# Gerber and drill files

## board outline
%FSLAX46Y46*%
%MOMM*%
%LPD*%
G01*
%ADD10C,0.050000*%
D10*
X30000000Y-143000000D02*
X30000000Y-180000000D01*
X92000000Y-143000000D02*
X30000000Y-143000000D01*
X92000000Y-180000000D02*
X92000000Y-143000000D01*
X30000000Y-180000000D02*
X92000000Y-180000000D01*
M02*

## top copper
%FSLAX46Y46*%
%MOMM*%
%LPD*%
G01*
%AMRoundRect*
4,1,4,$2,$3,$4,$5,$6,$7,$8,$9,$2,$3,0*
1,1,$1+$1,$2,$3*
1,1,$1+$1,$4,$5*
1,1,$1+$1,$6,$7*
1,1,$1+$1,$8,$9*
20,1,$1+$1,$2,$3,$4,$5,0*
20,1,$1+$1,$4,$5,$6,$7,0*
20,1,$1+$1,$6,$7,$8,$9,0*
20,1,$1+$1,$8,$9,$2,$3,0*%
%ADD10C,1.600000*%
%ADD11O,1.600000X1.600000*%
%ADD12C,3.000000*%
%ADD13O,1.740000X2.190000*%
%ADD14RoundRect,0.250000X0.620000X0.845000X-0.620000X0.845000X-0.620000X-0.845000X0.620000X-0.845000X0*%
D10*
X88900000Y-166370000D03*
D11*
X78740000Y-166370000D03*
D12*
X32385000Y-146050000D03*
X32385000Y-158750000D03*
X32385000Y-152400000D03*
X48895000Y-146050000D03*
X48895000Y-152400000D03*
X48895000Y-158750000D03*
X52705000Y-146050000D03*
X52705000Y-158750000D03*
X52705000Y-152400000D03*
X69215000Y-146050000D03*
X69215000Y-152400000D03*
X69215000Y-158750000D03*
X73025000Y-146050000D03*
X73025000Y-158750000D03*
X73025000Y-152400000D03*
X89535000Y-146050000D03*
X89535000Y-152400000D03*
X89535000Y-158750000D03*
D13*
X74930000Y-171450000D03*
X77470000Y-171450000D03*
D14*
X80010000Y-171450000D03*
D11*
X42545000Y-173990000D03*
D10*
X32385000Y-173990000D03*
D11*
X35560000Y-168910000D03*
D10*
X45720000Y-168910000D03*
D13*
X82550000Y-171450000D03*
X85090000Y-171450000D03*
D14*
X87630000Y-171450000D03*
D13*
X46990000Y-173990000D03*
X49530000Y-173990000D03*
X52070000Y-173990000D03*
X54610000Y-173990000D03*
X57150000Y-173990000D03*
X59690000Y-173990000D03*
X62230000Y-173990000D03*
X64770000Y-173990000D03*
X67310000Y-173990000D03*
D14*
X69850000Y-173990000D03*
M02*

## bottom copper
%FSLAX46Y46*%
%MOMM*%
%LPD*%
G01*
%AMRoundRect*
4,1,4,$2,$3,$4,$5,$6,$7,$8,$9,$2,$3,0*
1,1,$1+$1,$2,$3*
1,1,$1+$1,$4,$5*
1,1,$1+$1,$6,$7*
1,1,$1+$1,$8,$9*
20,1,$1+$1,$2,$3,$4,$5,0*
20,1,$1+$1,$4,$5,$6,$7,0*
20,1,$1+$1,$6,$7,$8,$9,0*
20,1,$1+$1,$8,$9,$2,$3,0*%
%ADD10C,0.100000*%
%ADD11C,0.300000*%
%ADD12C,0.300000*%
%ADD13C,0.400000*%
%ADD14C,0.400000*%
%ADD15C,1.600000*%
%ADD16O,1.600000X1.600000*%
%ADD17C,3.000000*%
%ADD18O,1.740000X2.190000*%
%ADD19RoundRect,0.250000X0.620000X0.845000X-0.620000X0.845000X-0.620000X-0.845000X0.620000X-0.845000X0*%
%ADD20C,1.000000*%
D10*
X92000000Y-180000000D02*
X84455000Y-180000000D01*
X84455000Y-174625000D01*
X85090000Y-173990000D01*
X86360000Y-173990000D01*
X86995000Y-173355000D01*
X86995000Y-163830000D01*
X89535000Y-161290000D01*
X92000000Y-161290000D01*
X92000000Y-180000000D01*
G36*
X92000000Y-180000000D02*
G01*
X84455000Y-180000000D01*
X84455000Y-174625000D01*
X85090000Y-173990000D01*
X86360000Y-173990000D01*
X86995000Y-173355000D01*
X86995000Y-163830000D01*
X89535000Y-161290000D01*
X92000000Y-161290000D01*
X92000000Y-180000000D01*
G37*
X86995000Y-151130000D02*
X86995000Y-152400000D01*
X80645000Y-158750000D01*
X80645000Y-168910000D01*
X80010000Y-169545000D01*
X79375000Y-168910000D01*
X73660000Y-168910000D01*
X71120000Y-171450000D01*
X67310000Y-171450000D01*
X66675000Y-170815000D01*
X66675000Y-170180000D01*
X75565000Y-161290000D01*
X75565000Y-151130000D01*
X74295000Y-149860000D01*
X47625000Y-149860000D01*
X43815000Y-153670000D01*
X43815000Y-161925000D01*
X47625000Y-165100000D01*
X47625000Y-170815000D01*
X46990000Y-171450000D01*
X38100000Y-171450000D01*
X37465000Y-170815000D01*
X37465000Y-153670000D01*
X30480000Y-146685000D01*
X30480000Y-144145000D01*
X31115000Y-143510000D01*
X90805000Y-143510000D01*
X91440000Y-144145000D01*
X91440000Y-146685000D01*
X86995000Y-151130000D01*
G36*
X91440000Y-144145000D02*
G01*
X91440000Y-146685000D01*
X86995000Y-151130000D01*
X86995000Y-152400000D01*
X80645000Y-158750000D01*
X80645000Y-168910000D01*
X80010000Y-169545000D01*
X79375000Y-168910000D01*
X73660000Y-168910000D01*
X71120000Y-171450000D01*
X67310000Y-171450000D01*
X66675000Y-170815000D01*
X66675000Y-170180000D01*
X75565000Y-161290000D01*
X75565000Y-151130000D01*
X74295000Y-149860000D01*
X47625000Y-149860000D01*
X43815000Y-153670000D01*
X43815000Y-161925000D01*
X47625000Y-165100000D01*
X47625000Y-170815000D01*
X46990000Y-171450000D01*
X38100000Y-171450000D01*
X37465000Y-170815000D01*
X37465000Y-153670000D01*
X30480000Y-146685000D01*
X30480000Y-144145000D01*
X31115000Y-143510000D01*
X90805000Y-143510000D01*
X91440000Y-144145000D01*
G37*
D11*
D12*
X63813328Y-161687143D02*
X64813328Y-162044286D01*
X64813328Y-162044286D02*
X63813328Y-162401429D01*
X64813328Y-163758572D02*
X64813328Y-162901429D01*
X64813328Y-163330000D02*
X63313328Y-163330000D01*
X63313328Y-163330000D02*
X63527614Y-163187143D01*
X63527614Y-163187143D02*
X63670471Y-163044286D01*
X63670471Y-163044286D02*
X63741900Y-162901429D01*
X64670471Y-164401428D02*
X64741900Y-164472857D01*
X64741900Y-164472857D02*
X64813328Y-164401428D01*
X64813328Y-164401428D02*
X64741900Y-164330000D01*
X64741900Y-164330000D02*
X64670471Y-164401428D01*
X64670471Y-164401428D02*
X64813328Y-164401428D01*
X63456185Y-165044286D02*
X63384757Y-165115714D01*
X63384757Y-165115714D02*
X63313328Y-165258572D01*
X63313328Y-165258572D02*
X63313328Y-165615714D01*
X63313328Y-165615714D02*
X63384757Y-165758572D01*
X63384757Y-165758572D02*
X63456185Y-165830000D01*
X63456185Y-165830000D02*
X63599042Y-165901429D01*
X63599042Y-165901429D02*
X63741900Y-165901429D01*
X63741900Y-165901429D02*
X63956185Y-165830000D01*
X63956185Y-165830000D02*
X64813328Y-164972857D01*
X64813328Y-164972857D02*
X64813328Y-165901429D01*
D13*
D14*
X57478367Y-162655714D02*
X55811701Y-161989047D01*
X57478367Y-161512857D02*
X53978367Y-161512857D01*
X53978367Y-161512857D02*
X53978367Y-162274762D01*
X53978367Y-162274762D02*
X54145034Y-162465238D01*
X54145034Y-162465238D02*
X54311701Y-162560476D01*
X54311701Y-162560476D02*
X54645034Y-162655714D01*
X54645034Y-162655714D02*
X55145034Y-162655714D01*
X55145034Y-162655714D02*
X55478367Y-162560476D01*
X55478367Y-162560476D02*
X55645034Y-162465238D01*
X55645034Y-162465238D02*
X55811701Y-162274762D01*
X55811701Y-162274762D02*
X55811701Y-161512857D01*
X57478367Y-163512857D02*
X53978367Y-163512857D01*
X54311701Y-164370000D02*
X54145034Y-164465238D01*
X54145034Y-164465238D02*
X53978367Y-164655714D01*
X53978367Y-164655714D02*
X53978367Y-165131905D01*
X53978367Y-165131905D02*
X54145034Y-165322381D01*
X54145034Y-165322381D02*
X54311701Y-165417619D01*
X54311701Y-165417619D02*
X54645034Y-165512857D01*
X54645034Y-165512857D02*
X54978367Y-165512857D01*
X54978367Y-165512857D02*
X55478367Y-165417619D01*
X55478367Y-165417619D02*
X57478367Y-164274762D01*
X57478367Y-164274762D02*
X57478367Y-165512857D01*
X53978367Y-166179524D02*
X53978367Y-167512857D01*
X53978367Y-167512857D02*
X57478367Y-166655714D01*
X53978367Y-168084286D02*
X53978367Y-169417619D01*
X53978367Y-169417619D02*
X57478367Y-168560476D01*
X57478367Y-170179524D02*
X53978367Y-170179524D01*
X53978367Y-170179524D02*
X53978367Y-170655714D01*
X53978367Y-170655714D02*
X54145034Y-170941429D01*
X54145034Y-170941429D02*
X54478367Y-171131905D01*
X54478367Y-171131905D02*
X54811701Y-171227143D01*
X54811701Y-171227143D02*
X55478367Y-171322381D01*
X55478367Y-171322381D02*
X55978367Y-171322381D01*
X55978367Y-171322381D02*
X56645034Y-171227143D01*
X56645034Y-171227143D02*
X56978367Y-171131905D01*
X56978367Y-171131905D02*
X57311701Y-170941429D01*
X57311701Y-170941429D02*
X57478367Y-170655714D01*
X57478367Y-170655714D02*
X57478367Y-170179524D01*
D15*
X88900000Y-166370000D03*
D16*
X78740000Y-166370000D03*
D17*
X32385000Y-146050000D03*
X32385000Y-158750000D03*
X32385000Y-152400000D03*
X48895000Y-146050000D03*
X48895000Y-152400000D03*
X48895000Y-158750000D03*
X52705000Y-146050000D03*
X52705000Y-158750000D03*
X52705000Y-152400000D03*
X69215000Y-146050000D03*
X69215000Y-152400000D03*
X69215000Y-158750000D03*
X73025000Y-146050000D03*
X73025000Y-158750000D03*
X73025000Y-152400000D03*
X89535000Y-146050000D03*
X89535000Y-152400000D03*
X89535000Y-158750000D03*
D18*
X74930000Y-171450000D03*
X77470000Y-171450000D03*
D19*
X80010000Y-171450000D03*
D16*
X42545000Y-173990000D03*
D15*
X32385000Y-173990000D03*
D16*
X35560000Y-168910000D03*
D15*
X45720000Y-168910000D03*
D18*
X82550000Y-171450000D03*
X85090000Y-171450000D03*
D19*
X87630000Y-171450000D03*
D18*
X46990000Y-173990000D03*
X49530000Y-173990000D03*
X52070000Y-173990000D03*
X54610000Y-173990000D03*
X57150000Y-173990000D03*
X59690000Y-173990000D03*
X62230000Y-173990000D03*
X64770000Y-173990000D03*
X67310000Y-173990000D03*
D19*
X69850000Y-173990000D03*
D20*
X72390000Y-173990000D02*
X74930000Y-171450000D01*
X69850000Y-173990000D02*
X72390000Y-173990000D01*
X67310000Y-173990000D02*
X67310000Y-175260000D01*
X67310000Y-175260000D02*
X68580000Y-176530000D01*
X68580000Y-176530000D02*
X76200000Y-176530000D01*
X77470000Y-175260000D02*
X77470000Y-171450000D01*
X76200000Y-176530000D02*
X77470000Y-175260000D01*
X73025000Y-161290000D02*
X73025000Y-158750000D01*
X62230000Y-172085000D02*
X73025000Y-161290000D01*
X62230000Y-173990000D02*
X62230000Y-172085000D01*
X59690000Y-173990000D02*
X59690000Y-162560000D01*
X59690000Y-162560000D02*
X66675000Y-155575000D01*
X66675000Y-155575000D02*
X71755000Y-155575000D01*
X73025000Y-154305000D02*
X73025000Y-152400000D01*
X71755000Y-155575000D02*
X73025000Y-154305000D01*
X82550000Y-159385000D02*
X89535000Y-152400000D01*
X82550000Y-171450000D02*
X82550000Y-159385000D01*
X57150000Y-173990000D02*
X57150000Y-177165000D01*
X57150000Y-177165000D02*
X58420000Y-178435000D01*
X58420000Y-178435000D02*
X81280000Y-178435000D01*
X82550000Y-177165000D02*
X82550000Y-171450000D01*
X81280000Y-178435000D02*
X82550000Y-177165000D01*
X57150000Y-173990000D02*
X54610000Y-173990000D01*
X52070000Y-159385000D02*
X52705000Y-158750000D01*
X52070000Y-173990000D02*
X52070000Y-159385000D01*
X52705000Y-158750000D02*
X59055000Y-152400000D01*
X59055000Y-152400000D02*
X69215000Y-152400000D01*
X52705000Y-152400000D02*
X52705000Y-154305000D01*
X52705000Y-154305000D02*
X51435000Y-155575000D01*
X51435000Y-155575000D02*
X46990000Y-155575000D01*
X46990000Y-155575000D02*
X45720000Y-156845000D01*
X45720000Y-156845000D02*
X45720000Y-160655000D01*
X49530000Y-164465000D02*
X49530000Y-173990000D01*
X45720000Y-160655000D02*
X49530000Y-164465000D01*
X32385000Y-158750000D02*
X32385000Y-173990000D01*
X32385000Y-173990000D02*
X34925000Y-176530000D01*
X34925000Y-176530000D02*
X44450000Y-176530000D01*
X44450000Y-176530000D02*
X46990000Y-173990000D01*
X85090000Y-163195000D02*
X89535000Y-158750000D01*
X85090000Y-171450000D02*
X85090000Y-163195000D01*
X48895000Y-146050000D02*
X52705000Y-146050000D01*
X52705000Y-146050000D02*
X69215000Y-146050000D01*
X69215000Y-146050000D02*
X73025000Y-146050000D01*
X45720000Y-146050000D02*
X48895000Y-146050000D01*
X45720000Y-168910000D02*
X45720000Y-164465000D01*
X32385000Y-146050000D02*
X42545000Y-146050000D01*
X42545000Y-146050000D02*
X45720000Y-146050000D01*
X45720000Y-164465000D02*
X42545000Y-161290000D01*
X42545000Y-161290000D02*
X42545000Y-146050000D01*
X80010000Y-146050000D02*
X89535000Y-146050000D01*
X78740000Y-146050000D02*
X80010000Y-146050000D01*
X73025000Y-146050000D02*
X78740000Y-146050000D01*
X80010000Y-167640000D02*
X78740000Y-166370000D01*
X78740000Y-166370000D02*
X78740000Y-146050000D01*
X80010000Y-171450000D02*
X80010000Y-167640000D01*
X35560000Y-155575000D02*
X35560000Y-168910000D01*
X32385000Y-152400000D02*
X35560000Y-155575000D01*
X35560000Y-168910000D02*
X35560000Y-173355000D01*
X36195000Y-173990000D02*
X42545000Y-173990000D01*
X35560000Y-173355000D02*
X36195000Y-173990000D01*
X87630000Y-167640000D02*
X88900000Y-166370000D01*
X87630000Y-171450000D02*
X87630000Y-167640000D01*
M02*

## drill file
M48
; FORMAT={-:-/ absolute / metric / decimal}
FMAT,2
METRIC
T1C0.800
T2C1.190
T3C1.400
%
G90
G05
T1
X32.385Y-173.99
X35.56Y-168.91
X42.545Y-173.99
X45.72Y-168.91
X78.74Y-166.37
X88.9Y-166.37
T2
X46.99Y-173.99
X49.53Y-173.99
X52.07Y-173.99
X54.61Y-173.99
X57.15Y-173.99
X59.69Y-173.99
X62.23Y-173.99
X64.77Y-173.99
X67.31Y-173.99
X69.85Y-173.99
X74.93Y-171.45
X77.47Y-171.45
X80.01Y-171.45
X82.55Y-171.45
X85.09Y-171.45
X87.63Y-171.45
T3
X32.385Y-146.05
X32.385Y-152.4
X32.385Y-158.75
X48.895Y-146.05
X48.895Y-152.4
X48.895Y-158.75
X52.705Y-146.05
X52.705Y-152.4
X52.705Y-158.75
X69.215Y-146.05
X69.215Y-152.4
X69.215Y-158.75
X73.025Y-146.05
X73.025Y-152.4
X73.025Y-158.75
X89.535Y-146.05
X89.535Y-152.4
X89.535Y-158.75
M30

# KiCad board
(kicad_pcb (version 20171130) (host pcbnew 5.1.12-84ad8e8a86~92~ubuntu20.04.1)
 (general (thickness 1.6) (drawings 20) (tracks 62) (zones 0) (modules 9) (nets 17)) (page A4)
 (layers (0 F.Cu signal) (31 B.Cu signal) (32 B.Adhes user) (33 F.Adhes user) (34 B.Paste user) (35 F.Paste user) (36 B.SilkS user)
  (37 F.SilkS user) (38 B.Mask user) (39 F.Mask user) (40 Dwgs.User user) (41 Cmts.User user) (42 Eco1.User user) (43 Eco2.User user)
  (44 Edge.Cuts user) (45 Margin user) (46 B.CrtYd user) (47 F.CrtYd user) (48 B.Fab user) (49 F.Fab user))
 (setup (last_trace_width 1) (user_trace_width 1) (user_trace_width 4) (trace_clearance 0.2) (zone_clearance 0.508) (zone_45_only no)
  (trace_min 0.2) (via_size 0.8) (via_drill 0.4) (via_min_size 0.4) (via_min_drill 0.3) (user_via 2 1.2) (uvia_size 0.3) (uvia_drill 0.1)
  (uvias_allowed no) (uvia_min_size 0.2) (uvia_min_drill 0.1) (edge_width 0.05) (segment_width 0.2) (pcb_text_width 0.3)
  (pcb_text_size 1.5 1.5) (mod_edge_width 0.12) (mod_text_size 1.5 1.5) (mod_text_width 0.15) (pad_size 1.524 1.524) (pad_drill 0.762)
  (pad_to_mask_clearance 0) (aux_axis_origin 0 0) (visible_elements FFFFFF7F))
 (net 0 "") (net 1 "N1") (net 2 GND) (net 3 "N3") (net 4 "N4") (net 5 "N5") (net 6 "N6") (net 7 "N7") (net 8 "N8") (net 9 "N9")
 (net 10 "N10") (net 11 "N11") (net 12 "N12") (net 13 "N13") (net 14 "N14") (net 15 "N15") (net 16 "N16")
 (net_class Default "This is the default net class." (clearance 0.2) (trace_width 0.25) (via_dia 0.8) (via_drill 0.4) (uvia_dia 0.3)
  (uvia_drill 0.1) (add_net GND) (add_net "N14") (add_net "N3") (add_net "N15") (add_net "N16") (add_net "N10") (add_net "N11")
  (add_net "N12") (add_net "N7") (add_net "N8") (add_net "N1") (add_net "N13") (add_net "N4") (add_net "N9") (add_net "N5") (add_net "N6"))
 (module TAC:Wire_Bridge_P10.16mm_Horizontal (layer F.Cu) (at 88.9 166.37 180)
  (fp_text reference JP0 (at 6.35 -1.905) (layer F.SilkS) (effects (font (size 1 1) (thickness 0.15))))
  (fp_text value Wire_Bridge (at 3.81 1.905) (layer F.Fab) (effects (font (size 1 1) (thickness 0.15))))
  (pad 1 thru_hole circle (at 0 0 180) (size 1.6 1.6) (drill 0.8) (layers *.Cu *.Mask) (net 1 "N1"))
  (pad 2 thru_hole oval (at 10.16 0 180) (size 1.6 1.6) (drill 0.8) (layers *.Cu *.Mask) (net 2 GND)))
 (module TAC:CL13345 (layer F.Cu) (at 40.64 146.05 90)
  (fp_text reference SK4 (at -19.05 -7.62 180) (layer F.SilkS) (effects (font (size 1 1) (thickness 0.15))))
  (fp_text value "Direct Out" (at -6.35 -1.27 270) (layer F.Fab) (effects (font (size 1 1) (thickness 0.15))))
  (pad S thru_hole circle (at 0 -8.255 180) (size 3 3) (drill 1.4) (layers *.Cu *.Mask) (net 2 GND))
  (pad T thru_hole circle (at -12.7 -8.255 180) (size 3 3) (drill 1.4) (layers *.Cu *.Mask) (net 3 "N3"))
  (pad R thru_hole circle (at -6.35 -8.255 180) (size 3 3) (drill 1.4) (layers *.Cu *.Mask) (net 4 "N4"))
  (pad SN thru_hole circle (at 0 8.255 180) (size 3 3) (drill 1.4) (layers *.Cu *.Mask) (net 2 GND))
  (pad RN thru_hole circle (at -6.35 8.255 180) (size 3 3) (drill 1.4) (layers *.Cu *.Mask) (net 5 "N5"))
  (pad TN thru_hole circle (at -12.7 8.255 180) (size 3 3) (drill 1.4) (layers *.Cu *.Mask) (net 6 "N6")))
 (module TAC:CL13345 (layer F.Cu) (at 60.96 146.05 90)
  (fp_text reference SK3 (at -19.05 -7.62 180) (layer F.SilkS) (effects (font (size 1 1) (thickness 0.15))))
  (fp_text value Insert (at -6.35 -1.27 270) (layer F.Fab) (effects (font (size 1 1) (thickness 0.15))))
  (pad S thru_hole circle (at 0 -8.255 180) (size 3 3) (drill 1.4) (layers *.Cu *.Mask) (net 2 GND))
  (pad T thru_hole circle (at -12.7 -8.255 180) (size 3 3) (drill 1.4) (layers *.Cu *.Mask) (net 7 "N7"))
  (pad R thru_hole circle (at -6.35 -8.255 180) (size 3 3) (drill 1.4) (layers *.Cu *.Mask) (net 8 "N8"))
  (pad SN thru_hole circle (at 0 8.255 180) (size 3 3) (drill 1.4) (layers *.Cu *.Mask) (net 2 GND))
  (pad RN thru_hole circle (at -6.35 8.255 180) (size 3 3) (drill 1.4) (layers *.Cu *.Mask) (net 7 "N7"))
  (pad TN thru_hole circle (at -12.7 8.255 180) (size 3 3) (drill 1.4) (layers *.Cu *.Mask) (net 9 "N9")))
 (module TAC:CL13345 (layer F.Cu) (at 81.28 146.05 90)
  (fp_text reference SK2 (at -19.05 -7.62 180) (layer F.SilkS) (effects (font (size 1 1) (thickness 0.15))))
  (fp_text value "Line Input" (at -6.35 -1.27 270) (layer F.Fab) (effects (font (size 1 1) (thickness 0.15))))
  (pad S thru_hole circle (at 0 -8.255 180) (size 3 3) (drill 1.4) (layers *.Cu *.Mask) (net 2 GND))
  (pad T thru_hole circle (at -12.7 -8.255 180) (size 3 3) (drill 1.4) (layers *.Cu *.Mask) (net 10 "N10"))
  (pad R thru_hole circle (at -6.35 -8.255 180) (size 3 3) (drill 1.4) (layers *.Cu *.Mask) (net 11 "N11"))
  (pad SN thru_hole circle (at 0 8.255 180) (size 3 3) (drill 1.4) (layers *.Cu *.Mask) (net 2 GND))
  (pad RN thru_hole circle (at -6.35 8.255 180) (size 3 3) (drill 1.4) (layers *.Cu *.Mask) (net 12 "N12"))
  (pad TN thru_hole circle (at -12.7 8.255 180) (size 3 3) (drill 1.4) (layers *.Cu *.Mask) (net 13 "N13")))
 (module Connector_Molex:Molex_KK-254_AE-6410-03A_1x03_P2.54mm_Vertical (layer F.Cu) (at 80.01 171.45 180)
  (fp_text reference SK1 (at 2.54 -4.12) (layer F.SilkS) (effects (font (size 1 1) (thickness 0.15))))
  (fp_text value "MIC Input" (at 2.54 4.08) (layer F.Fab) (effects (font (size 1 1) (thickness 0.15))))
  (pad 3 thru_hole oval (at 5.08 0 180) (size 1.74 2.19) (drill 1.19) (layers *.Cu *.Mask) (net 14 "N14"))
  (pad 2 thru_hole oval (at 2.54 0 180) (size 1.74 2.19) (drill 1.19) (layers *.Cu *.Mask) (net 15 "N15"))
  (pad 1 thru_hole roundrect (at 0 0 180) (size 1.74 2.19) (drill 1.19) (layers *.Cu *.Mask) (roundrect_rratio 0.143678) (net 2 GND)))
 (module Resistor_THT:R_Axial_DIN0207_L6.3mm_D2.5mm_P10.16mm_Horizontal (layer F.Cu) (at 32.385 173.99)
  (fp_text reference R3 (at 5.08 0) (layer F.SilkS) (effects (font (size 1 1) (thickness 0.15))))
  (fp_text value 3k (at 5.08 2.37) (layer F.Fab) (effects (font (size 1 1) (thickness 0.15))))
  (pad 2 thru_hole oval (at 10.16 0) (size 1.6 1.6) (drill 0.8) (layers *.Cu *.Mask) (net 4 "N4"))
  (pad 1 thru_hole circle (at 0 0) (size 1.6 1.6) (drill 0.8) (layers *.Cu *.Mask) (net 3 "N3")))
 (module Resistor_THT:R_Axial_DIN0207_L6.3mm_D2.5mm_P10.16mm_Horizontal (layer F.Cu) (at 45.72 168.91 180)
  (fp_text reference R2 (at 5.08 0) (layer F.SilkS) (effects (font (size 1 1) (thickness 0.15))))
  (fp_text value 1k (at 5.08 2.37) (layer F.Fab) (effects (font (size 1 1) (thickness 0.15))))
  (pad 2 thru_hole oval (at 10.16 0 180) (size 1.6 1.6) (drill 0.8) (layers *.Cu *.Mask) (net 4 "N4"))
  (pad 1 thru_hole circle (at 0 0 180) (size 1.6 1.6) (drill 0.8) (layers *.Cu *.Mask) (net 2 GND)))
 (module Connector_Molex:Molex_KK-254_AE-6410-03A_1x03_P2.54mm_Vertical (layer F.Cu) (at 87.63 171.45 180)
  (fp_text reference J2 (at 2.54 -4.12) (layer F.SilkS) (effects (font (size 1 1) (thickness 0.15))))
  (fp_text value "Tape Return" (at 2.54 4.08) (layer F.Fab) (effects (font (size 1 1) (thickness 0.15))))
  (pad 3 thru_hole oval (at 5.08 0 180) (size 1.74 2.19) (drill 1.19) (layers *.Cu *.Mask) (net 12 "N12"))
  (pad 2 thru_hole oval (at 2.54 0 180) (size 1.74 2.19) (drill 1.19) (layers *.Cu *.Mask) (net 13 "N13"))
  (pad 1 thru_hole roundrect (at 0 0 180) (size 1.74 2.19) (drill 1.19) (layers *.Cu *.Mask) (roundrect_rratio 0.143678) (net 1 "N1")))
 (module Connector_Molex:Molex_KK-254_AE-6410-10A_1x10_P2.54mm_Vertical (layer F.Cu) (at 69.85 173.99 180)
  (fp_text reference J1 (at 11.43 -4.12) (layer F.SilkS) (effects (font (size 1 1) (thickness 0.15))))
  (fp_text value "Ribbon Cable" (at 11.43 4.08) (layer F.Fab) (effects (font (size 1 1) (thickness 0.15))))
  (pad 10 thru_hole oval (at 22.86 0 180) (size 1.74 2.19) (drill 1.19) (layers *.Cu *.Mask) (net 3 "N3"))
  (pad 9 thru_hole oval (at 20.32 0 180) (size 1.74 2.19) (drill 1.19) (layers *.Cu *.Mask) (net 8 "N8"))
  (pad 8 thru_hole oval (at 17.78 0 180) (size 1.74 2.19) (drill 1.19) (layers *.Cu *.Mask) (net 7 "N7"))
  (pad 7 thru_hole oval (at 15.24 0 180) (size 1.74 2.19) (drill 1.19) (layers *.Cu *.Mask) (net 12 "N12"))
  (pad 6 thru_hole oval (at 12.7 0 180) (size 1.74 2.19) (drill 1.19) (layers *.Cu *.Mask) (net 12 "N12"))
  (pad 5 thru_hole oval (at 10.16 0 180) (size 1.74 2.19) (drill 1.19) (layers *.Cu *.Mask) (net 11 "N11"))
  (pad 4 thru_hole oval (at 7.62 0 180) (size 1.74 2.19) (drill 1.19) (layers *.Cu *.Mask) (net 10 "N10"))
  (pad 3 thru_hole oval (at 5.08 0 180) (size 1.74 2.19) (drill 1.19) (layers *.Cu *.Mask) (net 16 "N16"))
  (pad 2 thru_hole oval (at 2.54 0 180) (size 1.74 2.19) (drill 1.19) (layers *.Cu *.Mask) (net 15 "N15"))
  (pad 1 thru_hole roundrect (at 0 0 180) (size 1.74 2.19) (drill 1.19) (layers *.Cu *.Mask) (roundrect_rratio 0.143678) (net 14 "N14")))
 (gr_poly
  (pts (xy 92 180) (xy 84.455 180) (xy 84.455 174.625) (xy 85.09 173.99) (xy 86.36 173.99) (xy 86.995 173.355) (xy 86.995 163.83)
   (xy 89.535 161.29) (xy 92 161.29))
  (layer B.Cu) (width 0.1))
 (gr_poly
  (pts (xy 86.995 151.13) (xy 86.995 152.4) (xy 80.645 158.75) (xy 80.645 168.91) (xy 80.01 169.545) (xy 79.375 168.91) (xy 73.66 168.91)
   (xy 71.12 171.45) (xy 67.31 171.45) (xy 66.675 170.815) (xy 66.675 170.18) (xy 75.565 161.29) (xy 75.565 151.13) (xy 74.295 149.86)
   (xy 47.625 149.86) (xy 43.815 153.67) (xy 43.815 161.925) (xy 47.625 165.1) (xy 47.625 170.815) (xy 46.99 171.45) (xy 38.1 171.45)
   (xy 37.465 170.815) (xy 37.465 153.67) (xy 30.48 146.685) (xy 30.48 144.145) (xy 31.115 143.51) (xy 90.805 143.51) (xy 91.44 144.145)
   (xy 91.44 146.685))
  (layer B.Cu) (width 0.1))
 (gr_line (start 30 143) (end 30 180) (layer Edge.Cuts) (width 0.05))
 (gr_line (start 92 143) (end 30 143) (layer Edge.Cuts) (width 0.05))
 (gr_line (start 92 180) (end 92 143) (layer Edge.Cuts) (width 0.05))
 (gr_line (start 30 180) (end 92 180) (layer Edge.Cuts) (width 0.05))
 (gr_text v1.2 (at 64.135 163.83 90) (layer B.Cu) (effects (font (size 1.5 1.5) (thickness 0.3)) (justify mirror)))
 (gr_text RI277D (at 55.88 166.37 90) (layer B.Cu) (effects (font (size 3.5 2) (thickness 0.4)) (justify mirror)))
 (segment (start 72.39 173.99) (end 74.93 171.45) (width 1) (layer B.Cu) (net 14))
 (segment (start 69.85 173.99) (end 72.39 173.99) (width 1) (layer B.Cu) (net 14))
 (segment (start 67.31 173.99) (end 67.31 175.26) (width 1) (layer B.Cu) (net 15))
 (segment (start 67.31 175.26) (end 68.58 176.53) (width 1) (layer B.Cu) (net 15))
 (segment (start 68.58 176.53) (end 76.2 176.53) (width 1) (layer B.Cu) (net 15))
 (segment (start 77.47 175.26) (end 77.47 171.45) (width 1) (layer B.Cu) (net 15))
 (segment (start 76.2 176.53) (end 77.47 175.26) (width 1) (layer B.Cu) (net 15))
 (segment (start 73.025 161.29) (end 73.025 158.75) (width 1) (layer B.Cu) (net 10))
 (segment (start 62.23 172.085) (end 73.025 161.29) (width 1) (layer B.Cu) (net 10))
 (segment (start 62.23 173.99) (end 62.23 172.085) (width 1) (layer B.Cu) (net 10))
 (segment (start 59.69 173.99) (end 59.69 162.56) (width 1) (layer B.Cu) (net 11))
 (segment (start 59.69 162.56) (end 66.675 155.575) (width 1) (layer B.Cu) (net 11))
 (segment (start 66.675 155.575) (end 71.755 155.575) (width 1) (layer B.Cu) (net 11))
 (segment (start 73.025 154.305) (end 73.025 152.4) (width 1) (layer B.Cu) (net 11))
 (segment (start 71.755 155.575) (end 73.025 154.305) (width 1) (layer B.Cu) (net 11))
 (segment (start 82.55 159.385) (end 89.535 152.4) (width 1) (layer B.Cu) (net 12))
 (segment (start 82.55 171.45) (end 82.55 159.385) (width 1) (layer B.Cu) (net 12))
 (segment (start 57.15 173.99) (end 57.15 177.165) (width 1) (layer B.Cu) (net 12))
 (segment (start 57.15 177.165) (end 58.42 178.435) (width 1) (layer B.Cu) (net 12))
 (segment (start 58.42 178.435) (end 81.28 178.435) (width 1) (layer B.Cu) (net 12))
 (segment (start 82.55 177.165) (end 82.55 171.45) (width 1) (layer B.Cu) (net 12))
 (segment (start 81.28 178.435) (end 82.55 177.165) (width 1) (layer B.Cu) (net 12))
 (segment (start 57.15 173.99) (end 54.61 173.99) (width 1) (layer B.Cu) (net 12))
 (segment (start 52.07 159.385) (end 52.705 158.75) (width 1) (layer B.Cu) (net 7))
 (segment (start 52.07 173.99) (end 52.07 159.385) (width 1) (layer B.Cu) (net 7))
 (segment (start 52.705 158.75) (end 59.055 152.4) (width 1) (layer B.Cu) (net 7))
 (segment (start 59.055 152.4) (end 69.215 152.4) (width 1) (layer B.Cu) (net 7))
 (segment (start 52.705 152.4) (end 52.705 154.305) (width 1) (layer B.Cu) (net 8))
 (segment (start 52.705 154.305) (end 51.435 155.575) (width 1) (layer B.Cu) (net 8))
 (segment (start 51.435 155.575) (end 46.99 155.575) (width 1) (layer B.Cu) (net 8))
 (segment (start 46.99 155.575) (end 45.72 156.845) (width 1) (layer B.Cu) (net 8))
 (segment (start 45.72 156.845) (end 45.72 160.655) (width 1) (layer B.Cu) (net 8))
 (segment (start 49.53 164.465) (end 49.53 173.99) (width 1) (layer B.Cu) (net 8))
 (segment (start 45.72 160.655) (end 49.53 164.465) (width 1) (layer B.Cu) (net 8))
 (segment (start 32.385 158.75) (end 32.385 173.99) (width 1) (layer B.Cu) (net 3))
 (segment (start 32.385 173.99) (end 34.925 176.53) (width 1) (layer B.Cu) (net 3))
 (segment (start 34.925 176.53) (end 44.45 176.53) (width 1) (layer B.Cu) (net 3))
 (segment (start 44.45 176.53) (end 46.99 173.99) (width 1) (layer B.Cu) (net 3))
 (segment (start 85.09 163.195) (end 89.535 158.75) (width 1) (layer B.Cu) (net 13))
 (segment (start 85.09 171.45) (end 85.09 163.195) (width 1) (layer B.Cu) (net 13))
 (segment (start 48.895 146.05) (end 52.705 146.05) (width 1) (layer B.Cu) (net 2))
 (segment (start 52.705 146.05) (end 69.215 146.05) (width 1) (layer B.Cu) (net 2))
 (segment (start 69.215 146.05) (end 73.025 146.05) (width 1) (layer B.Cu) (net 2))
 (segment (start 45.72 146.05) (end 48.895 146.05) (width 1) (layer B.Cu) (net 2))
 (segment (start 45.72 168.91) (end 45.72 164.465) (width 1) (layer B.Cu) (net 2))
 (segment (start 32.385 146.05) (end 42.545 146.05) (width 1) (layer B.Cu) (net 2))
 (segment (start 42.545 146.05) (end 45.72 146.05) (width 1) (layer B.Cu) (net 2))
 (segment (start 45.72 164.465) (end 42.545 161.29) (width 1) (layer B.Cu) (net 2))
 (segment (start 42.545 161.29) (end 42.545 146.05) (width 1) (layer B.Cu) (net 2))
 (segment (start 80.01 146.05) (end 89.535 146.05) (width 1) (layer B.Cu) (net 2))
 (segment (start 78.74 146.05) (end 80.01 146.05) (width 1) (layer B.Cu) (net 2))
 (segment (start 73.025 146.05) (end 78.74 146.05) (width 1) (layer B.Cu) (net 2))
 (segment (start 80.01 167.64) (end 78.74 166.37) (width 1) (layer B.Cu) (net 2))
 (segment (start 78.74 166.37) (end 78.74 146.05) (width 1) (layer B.Cu) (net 2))
 (segment (start 80.01 171.45) (end 80.01 167.64) (width 1) (layer B.Cu) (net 2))
 (segment (start 35.56 155.575) (end 35.56 168.91) (width 1) (layer B.Cu) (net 4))
 (segment (start 32.385 152.4) (end 35.56 155.575) (width 1) (layer B.Cu) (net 4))
 (segment (start 35.56 168.91) (end 35.56 173.355) (width 1) (layer B.Cu) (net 4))
 (segment (start 36.195 173.99) (end 42.545 173.99) (width 1) (layer B.Cu) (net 4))
 (segment (start 35.56 173.355) (end 36.195 173.99) (width 1) (layer B.Cu) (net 4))
 (segment (start 87.63 167.64) (end 88.9 166.37) (width 1) (layer B.Cu) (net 1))
 (segment (start 87.63 171.45) (end 87.63 167.64) (width 1) (layer B.Cu) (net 1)))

